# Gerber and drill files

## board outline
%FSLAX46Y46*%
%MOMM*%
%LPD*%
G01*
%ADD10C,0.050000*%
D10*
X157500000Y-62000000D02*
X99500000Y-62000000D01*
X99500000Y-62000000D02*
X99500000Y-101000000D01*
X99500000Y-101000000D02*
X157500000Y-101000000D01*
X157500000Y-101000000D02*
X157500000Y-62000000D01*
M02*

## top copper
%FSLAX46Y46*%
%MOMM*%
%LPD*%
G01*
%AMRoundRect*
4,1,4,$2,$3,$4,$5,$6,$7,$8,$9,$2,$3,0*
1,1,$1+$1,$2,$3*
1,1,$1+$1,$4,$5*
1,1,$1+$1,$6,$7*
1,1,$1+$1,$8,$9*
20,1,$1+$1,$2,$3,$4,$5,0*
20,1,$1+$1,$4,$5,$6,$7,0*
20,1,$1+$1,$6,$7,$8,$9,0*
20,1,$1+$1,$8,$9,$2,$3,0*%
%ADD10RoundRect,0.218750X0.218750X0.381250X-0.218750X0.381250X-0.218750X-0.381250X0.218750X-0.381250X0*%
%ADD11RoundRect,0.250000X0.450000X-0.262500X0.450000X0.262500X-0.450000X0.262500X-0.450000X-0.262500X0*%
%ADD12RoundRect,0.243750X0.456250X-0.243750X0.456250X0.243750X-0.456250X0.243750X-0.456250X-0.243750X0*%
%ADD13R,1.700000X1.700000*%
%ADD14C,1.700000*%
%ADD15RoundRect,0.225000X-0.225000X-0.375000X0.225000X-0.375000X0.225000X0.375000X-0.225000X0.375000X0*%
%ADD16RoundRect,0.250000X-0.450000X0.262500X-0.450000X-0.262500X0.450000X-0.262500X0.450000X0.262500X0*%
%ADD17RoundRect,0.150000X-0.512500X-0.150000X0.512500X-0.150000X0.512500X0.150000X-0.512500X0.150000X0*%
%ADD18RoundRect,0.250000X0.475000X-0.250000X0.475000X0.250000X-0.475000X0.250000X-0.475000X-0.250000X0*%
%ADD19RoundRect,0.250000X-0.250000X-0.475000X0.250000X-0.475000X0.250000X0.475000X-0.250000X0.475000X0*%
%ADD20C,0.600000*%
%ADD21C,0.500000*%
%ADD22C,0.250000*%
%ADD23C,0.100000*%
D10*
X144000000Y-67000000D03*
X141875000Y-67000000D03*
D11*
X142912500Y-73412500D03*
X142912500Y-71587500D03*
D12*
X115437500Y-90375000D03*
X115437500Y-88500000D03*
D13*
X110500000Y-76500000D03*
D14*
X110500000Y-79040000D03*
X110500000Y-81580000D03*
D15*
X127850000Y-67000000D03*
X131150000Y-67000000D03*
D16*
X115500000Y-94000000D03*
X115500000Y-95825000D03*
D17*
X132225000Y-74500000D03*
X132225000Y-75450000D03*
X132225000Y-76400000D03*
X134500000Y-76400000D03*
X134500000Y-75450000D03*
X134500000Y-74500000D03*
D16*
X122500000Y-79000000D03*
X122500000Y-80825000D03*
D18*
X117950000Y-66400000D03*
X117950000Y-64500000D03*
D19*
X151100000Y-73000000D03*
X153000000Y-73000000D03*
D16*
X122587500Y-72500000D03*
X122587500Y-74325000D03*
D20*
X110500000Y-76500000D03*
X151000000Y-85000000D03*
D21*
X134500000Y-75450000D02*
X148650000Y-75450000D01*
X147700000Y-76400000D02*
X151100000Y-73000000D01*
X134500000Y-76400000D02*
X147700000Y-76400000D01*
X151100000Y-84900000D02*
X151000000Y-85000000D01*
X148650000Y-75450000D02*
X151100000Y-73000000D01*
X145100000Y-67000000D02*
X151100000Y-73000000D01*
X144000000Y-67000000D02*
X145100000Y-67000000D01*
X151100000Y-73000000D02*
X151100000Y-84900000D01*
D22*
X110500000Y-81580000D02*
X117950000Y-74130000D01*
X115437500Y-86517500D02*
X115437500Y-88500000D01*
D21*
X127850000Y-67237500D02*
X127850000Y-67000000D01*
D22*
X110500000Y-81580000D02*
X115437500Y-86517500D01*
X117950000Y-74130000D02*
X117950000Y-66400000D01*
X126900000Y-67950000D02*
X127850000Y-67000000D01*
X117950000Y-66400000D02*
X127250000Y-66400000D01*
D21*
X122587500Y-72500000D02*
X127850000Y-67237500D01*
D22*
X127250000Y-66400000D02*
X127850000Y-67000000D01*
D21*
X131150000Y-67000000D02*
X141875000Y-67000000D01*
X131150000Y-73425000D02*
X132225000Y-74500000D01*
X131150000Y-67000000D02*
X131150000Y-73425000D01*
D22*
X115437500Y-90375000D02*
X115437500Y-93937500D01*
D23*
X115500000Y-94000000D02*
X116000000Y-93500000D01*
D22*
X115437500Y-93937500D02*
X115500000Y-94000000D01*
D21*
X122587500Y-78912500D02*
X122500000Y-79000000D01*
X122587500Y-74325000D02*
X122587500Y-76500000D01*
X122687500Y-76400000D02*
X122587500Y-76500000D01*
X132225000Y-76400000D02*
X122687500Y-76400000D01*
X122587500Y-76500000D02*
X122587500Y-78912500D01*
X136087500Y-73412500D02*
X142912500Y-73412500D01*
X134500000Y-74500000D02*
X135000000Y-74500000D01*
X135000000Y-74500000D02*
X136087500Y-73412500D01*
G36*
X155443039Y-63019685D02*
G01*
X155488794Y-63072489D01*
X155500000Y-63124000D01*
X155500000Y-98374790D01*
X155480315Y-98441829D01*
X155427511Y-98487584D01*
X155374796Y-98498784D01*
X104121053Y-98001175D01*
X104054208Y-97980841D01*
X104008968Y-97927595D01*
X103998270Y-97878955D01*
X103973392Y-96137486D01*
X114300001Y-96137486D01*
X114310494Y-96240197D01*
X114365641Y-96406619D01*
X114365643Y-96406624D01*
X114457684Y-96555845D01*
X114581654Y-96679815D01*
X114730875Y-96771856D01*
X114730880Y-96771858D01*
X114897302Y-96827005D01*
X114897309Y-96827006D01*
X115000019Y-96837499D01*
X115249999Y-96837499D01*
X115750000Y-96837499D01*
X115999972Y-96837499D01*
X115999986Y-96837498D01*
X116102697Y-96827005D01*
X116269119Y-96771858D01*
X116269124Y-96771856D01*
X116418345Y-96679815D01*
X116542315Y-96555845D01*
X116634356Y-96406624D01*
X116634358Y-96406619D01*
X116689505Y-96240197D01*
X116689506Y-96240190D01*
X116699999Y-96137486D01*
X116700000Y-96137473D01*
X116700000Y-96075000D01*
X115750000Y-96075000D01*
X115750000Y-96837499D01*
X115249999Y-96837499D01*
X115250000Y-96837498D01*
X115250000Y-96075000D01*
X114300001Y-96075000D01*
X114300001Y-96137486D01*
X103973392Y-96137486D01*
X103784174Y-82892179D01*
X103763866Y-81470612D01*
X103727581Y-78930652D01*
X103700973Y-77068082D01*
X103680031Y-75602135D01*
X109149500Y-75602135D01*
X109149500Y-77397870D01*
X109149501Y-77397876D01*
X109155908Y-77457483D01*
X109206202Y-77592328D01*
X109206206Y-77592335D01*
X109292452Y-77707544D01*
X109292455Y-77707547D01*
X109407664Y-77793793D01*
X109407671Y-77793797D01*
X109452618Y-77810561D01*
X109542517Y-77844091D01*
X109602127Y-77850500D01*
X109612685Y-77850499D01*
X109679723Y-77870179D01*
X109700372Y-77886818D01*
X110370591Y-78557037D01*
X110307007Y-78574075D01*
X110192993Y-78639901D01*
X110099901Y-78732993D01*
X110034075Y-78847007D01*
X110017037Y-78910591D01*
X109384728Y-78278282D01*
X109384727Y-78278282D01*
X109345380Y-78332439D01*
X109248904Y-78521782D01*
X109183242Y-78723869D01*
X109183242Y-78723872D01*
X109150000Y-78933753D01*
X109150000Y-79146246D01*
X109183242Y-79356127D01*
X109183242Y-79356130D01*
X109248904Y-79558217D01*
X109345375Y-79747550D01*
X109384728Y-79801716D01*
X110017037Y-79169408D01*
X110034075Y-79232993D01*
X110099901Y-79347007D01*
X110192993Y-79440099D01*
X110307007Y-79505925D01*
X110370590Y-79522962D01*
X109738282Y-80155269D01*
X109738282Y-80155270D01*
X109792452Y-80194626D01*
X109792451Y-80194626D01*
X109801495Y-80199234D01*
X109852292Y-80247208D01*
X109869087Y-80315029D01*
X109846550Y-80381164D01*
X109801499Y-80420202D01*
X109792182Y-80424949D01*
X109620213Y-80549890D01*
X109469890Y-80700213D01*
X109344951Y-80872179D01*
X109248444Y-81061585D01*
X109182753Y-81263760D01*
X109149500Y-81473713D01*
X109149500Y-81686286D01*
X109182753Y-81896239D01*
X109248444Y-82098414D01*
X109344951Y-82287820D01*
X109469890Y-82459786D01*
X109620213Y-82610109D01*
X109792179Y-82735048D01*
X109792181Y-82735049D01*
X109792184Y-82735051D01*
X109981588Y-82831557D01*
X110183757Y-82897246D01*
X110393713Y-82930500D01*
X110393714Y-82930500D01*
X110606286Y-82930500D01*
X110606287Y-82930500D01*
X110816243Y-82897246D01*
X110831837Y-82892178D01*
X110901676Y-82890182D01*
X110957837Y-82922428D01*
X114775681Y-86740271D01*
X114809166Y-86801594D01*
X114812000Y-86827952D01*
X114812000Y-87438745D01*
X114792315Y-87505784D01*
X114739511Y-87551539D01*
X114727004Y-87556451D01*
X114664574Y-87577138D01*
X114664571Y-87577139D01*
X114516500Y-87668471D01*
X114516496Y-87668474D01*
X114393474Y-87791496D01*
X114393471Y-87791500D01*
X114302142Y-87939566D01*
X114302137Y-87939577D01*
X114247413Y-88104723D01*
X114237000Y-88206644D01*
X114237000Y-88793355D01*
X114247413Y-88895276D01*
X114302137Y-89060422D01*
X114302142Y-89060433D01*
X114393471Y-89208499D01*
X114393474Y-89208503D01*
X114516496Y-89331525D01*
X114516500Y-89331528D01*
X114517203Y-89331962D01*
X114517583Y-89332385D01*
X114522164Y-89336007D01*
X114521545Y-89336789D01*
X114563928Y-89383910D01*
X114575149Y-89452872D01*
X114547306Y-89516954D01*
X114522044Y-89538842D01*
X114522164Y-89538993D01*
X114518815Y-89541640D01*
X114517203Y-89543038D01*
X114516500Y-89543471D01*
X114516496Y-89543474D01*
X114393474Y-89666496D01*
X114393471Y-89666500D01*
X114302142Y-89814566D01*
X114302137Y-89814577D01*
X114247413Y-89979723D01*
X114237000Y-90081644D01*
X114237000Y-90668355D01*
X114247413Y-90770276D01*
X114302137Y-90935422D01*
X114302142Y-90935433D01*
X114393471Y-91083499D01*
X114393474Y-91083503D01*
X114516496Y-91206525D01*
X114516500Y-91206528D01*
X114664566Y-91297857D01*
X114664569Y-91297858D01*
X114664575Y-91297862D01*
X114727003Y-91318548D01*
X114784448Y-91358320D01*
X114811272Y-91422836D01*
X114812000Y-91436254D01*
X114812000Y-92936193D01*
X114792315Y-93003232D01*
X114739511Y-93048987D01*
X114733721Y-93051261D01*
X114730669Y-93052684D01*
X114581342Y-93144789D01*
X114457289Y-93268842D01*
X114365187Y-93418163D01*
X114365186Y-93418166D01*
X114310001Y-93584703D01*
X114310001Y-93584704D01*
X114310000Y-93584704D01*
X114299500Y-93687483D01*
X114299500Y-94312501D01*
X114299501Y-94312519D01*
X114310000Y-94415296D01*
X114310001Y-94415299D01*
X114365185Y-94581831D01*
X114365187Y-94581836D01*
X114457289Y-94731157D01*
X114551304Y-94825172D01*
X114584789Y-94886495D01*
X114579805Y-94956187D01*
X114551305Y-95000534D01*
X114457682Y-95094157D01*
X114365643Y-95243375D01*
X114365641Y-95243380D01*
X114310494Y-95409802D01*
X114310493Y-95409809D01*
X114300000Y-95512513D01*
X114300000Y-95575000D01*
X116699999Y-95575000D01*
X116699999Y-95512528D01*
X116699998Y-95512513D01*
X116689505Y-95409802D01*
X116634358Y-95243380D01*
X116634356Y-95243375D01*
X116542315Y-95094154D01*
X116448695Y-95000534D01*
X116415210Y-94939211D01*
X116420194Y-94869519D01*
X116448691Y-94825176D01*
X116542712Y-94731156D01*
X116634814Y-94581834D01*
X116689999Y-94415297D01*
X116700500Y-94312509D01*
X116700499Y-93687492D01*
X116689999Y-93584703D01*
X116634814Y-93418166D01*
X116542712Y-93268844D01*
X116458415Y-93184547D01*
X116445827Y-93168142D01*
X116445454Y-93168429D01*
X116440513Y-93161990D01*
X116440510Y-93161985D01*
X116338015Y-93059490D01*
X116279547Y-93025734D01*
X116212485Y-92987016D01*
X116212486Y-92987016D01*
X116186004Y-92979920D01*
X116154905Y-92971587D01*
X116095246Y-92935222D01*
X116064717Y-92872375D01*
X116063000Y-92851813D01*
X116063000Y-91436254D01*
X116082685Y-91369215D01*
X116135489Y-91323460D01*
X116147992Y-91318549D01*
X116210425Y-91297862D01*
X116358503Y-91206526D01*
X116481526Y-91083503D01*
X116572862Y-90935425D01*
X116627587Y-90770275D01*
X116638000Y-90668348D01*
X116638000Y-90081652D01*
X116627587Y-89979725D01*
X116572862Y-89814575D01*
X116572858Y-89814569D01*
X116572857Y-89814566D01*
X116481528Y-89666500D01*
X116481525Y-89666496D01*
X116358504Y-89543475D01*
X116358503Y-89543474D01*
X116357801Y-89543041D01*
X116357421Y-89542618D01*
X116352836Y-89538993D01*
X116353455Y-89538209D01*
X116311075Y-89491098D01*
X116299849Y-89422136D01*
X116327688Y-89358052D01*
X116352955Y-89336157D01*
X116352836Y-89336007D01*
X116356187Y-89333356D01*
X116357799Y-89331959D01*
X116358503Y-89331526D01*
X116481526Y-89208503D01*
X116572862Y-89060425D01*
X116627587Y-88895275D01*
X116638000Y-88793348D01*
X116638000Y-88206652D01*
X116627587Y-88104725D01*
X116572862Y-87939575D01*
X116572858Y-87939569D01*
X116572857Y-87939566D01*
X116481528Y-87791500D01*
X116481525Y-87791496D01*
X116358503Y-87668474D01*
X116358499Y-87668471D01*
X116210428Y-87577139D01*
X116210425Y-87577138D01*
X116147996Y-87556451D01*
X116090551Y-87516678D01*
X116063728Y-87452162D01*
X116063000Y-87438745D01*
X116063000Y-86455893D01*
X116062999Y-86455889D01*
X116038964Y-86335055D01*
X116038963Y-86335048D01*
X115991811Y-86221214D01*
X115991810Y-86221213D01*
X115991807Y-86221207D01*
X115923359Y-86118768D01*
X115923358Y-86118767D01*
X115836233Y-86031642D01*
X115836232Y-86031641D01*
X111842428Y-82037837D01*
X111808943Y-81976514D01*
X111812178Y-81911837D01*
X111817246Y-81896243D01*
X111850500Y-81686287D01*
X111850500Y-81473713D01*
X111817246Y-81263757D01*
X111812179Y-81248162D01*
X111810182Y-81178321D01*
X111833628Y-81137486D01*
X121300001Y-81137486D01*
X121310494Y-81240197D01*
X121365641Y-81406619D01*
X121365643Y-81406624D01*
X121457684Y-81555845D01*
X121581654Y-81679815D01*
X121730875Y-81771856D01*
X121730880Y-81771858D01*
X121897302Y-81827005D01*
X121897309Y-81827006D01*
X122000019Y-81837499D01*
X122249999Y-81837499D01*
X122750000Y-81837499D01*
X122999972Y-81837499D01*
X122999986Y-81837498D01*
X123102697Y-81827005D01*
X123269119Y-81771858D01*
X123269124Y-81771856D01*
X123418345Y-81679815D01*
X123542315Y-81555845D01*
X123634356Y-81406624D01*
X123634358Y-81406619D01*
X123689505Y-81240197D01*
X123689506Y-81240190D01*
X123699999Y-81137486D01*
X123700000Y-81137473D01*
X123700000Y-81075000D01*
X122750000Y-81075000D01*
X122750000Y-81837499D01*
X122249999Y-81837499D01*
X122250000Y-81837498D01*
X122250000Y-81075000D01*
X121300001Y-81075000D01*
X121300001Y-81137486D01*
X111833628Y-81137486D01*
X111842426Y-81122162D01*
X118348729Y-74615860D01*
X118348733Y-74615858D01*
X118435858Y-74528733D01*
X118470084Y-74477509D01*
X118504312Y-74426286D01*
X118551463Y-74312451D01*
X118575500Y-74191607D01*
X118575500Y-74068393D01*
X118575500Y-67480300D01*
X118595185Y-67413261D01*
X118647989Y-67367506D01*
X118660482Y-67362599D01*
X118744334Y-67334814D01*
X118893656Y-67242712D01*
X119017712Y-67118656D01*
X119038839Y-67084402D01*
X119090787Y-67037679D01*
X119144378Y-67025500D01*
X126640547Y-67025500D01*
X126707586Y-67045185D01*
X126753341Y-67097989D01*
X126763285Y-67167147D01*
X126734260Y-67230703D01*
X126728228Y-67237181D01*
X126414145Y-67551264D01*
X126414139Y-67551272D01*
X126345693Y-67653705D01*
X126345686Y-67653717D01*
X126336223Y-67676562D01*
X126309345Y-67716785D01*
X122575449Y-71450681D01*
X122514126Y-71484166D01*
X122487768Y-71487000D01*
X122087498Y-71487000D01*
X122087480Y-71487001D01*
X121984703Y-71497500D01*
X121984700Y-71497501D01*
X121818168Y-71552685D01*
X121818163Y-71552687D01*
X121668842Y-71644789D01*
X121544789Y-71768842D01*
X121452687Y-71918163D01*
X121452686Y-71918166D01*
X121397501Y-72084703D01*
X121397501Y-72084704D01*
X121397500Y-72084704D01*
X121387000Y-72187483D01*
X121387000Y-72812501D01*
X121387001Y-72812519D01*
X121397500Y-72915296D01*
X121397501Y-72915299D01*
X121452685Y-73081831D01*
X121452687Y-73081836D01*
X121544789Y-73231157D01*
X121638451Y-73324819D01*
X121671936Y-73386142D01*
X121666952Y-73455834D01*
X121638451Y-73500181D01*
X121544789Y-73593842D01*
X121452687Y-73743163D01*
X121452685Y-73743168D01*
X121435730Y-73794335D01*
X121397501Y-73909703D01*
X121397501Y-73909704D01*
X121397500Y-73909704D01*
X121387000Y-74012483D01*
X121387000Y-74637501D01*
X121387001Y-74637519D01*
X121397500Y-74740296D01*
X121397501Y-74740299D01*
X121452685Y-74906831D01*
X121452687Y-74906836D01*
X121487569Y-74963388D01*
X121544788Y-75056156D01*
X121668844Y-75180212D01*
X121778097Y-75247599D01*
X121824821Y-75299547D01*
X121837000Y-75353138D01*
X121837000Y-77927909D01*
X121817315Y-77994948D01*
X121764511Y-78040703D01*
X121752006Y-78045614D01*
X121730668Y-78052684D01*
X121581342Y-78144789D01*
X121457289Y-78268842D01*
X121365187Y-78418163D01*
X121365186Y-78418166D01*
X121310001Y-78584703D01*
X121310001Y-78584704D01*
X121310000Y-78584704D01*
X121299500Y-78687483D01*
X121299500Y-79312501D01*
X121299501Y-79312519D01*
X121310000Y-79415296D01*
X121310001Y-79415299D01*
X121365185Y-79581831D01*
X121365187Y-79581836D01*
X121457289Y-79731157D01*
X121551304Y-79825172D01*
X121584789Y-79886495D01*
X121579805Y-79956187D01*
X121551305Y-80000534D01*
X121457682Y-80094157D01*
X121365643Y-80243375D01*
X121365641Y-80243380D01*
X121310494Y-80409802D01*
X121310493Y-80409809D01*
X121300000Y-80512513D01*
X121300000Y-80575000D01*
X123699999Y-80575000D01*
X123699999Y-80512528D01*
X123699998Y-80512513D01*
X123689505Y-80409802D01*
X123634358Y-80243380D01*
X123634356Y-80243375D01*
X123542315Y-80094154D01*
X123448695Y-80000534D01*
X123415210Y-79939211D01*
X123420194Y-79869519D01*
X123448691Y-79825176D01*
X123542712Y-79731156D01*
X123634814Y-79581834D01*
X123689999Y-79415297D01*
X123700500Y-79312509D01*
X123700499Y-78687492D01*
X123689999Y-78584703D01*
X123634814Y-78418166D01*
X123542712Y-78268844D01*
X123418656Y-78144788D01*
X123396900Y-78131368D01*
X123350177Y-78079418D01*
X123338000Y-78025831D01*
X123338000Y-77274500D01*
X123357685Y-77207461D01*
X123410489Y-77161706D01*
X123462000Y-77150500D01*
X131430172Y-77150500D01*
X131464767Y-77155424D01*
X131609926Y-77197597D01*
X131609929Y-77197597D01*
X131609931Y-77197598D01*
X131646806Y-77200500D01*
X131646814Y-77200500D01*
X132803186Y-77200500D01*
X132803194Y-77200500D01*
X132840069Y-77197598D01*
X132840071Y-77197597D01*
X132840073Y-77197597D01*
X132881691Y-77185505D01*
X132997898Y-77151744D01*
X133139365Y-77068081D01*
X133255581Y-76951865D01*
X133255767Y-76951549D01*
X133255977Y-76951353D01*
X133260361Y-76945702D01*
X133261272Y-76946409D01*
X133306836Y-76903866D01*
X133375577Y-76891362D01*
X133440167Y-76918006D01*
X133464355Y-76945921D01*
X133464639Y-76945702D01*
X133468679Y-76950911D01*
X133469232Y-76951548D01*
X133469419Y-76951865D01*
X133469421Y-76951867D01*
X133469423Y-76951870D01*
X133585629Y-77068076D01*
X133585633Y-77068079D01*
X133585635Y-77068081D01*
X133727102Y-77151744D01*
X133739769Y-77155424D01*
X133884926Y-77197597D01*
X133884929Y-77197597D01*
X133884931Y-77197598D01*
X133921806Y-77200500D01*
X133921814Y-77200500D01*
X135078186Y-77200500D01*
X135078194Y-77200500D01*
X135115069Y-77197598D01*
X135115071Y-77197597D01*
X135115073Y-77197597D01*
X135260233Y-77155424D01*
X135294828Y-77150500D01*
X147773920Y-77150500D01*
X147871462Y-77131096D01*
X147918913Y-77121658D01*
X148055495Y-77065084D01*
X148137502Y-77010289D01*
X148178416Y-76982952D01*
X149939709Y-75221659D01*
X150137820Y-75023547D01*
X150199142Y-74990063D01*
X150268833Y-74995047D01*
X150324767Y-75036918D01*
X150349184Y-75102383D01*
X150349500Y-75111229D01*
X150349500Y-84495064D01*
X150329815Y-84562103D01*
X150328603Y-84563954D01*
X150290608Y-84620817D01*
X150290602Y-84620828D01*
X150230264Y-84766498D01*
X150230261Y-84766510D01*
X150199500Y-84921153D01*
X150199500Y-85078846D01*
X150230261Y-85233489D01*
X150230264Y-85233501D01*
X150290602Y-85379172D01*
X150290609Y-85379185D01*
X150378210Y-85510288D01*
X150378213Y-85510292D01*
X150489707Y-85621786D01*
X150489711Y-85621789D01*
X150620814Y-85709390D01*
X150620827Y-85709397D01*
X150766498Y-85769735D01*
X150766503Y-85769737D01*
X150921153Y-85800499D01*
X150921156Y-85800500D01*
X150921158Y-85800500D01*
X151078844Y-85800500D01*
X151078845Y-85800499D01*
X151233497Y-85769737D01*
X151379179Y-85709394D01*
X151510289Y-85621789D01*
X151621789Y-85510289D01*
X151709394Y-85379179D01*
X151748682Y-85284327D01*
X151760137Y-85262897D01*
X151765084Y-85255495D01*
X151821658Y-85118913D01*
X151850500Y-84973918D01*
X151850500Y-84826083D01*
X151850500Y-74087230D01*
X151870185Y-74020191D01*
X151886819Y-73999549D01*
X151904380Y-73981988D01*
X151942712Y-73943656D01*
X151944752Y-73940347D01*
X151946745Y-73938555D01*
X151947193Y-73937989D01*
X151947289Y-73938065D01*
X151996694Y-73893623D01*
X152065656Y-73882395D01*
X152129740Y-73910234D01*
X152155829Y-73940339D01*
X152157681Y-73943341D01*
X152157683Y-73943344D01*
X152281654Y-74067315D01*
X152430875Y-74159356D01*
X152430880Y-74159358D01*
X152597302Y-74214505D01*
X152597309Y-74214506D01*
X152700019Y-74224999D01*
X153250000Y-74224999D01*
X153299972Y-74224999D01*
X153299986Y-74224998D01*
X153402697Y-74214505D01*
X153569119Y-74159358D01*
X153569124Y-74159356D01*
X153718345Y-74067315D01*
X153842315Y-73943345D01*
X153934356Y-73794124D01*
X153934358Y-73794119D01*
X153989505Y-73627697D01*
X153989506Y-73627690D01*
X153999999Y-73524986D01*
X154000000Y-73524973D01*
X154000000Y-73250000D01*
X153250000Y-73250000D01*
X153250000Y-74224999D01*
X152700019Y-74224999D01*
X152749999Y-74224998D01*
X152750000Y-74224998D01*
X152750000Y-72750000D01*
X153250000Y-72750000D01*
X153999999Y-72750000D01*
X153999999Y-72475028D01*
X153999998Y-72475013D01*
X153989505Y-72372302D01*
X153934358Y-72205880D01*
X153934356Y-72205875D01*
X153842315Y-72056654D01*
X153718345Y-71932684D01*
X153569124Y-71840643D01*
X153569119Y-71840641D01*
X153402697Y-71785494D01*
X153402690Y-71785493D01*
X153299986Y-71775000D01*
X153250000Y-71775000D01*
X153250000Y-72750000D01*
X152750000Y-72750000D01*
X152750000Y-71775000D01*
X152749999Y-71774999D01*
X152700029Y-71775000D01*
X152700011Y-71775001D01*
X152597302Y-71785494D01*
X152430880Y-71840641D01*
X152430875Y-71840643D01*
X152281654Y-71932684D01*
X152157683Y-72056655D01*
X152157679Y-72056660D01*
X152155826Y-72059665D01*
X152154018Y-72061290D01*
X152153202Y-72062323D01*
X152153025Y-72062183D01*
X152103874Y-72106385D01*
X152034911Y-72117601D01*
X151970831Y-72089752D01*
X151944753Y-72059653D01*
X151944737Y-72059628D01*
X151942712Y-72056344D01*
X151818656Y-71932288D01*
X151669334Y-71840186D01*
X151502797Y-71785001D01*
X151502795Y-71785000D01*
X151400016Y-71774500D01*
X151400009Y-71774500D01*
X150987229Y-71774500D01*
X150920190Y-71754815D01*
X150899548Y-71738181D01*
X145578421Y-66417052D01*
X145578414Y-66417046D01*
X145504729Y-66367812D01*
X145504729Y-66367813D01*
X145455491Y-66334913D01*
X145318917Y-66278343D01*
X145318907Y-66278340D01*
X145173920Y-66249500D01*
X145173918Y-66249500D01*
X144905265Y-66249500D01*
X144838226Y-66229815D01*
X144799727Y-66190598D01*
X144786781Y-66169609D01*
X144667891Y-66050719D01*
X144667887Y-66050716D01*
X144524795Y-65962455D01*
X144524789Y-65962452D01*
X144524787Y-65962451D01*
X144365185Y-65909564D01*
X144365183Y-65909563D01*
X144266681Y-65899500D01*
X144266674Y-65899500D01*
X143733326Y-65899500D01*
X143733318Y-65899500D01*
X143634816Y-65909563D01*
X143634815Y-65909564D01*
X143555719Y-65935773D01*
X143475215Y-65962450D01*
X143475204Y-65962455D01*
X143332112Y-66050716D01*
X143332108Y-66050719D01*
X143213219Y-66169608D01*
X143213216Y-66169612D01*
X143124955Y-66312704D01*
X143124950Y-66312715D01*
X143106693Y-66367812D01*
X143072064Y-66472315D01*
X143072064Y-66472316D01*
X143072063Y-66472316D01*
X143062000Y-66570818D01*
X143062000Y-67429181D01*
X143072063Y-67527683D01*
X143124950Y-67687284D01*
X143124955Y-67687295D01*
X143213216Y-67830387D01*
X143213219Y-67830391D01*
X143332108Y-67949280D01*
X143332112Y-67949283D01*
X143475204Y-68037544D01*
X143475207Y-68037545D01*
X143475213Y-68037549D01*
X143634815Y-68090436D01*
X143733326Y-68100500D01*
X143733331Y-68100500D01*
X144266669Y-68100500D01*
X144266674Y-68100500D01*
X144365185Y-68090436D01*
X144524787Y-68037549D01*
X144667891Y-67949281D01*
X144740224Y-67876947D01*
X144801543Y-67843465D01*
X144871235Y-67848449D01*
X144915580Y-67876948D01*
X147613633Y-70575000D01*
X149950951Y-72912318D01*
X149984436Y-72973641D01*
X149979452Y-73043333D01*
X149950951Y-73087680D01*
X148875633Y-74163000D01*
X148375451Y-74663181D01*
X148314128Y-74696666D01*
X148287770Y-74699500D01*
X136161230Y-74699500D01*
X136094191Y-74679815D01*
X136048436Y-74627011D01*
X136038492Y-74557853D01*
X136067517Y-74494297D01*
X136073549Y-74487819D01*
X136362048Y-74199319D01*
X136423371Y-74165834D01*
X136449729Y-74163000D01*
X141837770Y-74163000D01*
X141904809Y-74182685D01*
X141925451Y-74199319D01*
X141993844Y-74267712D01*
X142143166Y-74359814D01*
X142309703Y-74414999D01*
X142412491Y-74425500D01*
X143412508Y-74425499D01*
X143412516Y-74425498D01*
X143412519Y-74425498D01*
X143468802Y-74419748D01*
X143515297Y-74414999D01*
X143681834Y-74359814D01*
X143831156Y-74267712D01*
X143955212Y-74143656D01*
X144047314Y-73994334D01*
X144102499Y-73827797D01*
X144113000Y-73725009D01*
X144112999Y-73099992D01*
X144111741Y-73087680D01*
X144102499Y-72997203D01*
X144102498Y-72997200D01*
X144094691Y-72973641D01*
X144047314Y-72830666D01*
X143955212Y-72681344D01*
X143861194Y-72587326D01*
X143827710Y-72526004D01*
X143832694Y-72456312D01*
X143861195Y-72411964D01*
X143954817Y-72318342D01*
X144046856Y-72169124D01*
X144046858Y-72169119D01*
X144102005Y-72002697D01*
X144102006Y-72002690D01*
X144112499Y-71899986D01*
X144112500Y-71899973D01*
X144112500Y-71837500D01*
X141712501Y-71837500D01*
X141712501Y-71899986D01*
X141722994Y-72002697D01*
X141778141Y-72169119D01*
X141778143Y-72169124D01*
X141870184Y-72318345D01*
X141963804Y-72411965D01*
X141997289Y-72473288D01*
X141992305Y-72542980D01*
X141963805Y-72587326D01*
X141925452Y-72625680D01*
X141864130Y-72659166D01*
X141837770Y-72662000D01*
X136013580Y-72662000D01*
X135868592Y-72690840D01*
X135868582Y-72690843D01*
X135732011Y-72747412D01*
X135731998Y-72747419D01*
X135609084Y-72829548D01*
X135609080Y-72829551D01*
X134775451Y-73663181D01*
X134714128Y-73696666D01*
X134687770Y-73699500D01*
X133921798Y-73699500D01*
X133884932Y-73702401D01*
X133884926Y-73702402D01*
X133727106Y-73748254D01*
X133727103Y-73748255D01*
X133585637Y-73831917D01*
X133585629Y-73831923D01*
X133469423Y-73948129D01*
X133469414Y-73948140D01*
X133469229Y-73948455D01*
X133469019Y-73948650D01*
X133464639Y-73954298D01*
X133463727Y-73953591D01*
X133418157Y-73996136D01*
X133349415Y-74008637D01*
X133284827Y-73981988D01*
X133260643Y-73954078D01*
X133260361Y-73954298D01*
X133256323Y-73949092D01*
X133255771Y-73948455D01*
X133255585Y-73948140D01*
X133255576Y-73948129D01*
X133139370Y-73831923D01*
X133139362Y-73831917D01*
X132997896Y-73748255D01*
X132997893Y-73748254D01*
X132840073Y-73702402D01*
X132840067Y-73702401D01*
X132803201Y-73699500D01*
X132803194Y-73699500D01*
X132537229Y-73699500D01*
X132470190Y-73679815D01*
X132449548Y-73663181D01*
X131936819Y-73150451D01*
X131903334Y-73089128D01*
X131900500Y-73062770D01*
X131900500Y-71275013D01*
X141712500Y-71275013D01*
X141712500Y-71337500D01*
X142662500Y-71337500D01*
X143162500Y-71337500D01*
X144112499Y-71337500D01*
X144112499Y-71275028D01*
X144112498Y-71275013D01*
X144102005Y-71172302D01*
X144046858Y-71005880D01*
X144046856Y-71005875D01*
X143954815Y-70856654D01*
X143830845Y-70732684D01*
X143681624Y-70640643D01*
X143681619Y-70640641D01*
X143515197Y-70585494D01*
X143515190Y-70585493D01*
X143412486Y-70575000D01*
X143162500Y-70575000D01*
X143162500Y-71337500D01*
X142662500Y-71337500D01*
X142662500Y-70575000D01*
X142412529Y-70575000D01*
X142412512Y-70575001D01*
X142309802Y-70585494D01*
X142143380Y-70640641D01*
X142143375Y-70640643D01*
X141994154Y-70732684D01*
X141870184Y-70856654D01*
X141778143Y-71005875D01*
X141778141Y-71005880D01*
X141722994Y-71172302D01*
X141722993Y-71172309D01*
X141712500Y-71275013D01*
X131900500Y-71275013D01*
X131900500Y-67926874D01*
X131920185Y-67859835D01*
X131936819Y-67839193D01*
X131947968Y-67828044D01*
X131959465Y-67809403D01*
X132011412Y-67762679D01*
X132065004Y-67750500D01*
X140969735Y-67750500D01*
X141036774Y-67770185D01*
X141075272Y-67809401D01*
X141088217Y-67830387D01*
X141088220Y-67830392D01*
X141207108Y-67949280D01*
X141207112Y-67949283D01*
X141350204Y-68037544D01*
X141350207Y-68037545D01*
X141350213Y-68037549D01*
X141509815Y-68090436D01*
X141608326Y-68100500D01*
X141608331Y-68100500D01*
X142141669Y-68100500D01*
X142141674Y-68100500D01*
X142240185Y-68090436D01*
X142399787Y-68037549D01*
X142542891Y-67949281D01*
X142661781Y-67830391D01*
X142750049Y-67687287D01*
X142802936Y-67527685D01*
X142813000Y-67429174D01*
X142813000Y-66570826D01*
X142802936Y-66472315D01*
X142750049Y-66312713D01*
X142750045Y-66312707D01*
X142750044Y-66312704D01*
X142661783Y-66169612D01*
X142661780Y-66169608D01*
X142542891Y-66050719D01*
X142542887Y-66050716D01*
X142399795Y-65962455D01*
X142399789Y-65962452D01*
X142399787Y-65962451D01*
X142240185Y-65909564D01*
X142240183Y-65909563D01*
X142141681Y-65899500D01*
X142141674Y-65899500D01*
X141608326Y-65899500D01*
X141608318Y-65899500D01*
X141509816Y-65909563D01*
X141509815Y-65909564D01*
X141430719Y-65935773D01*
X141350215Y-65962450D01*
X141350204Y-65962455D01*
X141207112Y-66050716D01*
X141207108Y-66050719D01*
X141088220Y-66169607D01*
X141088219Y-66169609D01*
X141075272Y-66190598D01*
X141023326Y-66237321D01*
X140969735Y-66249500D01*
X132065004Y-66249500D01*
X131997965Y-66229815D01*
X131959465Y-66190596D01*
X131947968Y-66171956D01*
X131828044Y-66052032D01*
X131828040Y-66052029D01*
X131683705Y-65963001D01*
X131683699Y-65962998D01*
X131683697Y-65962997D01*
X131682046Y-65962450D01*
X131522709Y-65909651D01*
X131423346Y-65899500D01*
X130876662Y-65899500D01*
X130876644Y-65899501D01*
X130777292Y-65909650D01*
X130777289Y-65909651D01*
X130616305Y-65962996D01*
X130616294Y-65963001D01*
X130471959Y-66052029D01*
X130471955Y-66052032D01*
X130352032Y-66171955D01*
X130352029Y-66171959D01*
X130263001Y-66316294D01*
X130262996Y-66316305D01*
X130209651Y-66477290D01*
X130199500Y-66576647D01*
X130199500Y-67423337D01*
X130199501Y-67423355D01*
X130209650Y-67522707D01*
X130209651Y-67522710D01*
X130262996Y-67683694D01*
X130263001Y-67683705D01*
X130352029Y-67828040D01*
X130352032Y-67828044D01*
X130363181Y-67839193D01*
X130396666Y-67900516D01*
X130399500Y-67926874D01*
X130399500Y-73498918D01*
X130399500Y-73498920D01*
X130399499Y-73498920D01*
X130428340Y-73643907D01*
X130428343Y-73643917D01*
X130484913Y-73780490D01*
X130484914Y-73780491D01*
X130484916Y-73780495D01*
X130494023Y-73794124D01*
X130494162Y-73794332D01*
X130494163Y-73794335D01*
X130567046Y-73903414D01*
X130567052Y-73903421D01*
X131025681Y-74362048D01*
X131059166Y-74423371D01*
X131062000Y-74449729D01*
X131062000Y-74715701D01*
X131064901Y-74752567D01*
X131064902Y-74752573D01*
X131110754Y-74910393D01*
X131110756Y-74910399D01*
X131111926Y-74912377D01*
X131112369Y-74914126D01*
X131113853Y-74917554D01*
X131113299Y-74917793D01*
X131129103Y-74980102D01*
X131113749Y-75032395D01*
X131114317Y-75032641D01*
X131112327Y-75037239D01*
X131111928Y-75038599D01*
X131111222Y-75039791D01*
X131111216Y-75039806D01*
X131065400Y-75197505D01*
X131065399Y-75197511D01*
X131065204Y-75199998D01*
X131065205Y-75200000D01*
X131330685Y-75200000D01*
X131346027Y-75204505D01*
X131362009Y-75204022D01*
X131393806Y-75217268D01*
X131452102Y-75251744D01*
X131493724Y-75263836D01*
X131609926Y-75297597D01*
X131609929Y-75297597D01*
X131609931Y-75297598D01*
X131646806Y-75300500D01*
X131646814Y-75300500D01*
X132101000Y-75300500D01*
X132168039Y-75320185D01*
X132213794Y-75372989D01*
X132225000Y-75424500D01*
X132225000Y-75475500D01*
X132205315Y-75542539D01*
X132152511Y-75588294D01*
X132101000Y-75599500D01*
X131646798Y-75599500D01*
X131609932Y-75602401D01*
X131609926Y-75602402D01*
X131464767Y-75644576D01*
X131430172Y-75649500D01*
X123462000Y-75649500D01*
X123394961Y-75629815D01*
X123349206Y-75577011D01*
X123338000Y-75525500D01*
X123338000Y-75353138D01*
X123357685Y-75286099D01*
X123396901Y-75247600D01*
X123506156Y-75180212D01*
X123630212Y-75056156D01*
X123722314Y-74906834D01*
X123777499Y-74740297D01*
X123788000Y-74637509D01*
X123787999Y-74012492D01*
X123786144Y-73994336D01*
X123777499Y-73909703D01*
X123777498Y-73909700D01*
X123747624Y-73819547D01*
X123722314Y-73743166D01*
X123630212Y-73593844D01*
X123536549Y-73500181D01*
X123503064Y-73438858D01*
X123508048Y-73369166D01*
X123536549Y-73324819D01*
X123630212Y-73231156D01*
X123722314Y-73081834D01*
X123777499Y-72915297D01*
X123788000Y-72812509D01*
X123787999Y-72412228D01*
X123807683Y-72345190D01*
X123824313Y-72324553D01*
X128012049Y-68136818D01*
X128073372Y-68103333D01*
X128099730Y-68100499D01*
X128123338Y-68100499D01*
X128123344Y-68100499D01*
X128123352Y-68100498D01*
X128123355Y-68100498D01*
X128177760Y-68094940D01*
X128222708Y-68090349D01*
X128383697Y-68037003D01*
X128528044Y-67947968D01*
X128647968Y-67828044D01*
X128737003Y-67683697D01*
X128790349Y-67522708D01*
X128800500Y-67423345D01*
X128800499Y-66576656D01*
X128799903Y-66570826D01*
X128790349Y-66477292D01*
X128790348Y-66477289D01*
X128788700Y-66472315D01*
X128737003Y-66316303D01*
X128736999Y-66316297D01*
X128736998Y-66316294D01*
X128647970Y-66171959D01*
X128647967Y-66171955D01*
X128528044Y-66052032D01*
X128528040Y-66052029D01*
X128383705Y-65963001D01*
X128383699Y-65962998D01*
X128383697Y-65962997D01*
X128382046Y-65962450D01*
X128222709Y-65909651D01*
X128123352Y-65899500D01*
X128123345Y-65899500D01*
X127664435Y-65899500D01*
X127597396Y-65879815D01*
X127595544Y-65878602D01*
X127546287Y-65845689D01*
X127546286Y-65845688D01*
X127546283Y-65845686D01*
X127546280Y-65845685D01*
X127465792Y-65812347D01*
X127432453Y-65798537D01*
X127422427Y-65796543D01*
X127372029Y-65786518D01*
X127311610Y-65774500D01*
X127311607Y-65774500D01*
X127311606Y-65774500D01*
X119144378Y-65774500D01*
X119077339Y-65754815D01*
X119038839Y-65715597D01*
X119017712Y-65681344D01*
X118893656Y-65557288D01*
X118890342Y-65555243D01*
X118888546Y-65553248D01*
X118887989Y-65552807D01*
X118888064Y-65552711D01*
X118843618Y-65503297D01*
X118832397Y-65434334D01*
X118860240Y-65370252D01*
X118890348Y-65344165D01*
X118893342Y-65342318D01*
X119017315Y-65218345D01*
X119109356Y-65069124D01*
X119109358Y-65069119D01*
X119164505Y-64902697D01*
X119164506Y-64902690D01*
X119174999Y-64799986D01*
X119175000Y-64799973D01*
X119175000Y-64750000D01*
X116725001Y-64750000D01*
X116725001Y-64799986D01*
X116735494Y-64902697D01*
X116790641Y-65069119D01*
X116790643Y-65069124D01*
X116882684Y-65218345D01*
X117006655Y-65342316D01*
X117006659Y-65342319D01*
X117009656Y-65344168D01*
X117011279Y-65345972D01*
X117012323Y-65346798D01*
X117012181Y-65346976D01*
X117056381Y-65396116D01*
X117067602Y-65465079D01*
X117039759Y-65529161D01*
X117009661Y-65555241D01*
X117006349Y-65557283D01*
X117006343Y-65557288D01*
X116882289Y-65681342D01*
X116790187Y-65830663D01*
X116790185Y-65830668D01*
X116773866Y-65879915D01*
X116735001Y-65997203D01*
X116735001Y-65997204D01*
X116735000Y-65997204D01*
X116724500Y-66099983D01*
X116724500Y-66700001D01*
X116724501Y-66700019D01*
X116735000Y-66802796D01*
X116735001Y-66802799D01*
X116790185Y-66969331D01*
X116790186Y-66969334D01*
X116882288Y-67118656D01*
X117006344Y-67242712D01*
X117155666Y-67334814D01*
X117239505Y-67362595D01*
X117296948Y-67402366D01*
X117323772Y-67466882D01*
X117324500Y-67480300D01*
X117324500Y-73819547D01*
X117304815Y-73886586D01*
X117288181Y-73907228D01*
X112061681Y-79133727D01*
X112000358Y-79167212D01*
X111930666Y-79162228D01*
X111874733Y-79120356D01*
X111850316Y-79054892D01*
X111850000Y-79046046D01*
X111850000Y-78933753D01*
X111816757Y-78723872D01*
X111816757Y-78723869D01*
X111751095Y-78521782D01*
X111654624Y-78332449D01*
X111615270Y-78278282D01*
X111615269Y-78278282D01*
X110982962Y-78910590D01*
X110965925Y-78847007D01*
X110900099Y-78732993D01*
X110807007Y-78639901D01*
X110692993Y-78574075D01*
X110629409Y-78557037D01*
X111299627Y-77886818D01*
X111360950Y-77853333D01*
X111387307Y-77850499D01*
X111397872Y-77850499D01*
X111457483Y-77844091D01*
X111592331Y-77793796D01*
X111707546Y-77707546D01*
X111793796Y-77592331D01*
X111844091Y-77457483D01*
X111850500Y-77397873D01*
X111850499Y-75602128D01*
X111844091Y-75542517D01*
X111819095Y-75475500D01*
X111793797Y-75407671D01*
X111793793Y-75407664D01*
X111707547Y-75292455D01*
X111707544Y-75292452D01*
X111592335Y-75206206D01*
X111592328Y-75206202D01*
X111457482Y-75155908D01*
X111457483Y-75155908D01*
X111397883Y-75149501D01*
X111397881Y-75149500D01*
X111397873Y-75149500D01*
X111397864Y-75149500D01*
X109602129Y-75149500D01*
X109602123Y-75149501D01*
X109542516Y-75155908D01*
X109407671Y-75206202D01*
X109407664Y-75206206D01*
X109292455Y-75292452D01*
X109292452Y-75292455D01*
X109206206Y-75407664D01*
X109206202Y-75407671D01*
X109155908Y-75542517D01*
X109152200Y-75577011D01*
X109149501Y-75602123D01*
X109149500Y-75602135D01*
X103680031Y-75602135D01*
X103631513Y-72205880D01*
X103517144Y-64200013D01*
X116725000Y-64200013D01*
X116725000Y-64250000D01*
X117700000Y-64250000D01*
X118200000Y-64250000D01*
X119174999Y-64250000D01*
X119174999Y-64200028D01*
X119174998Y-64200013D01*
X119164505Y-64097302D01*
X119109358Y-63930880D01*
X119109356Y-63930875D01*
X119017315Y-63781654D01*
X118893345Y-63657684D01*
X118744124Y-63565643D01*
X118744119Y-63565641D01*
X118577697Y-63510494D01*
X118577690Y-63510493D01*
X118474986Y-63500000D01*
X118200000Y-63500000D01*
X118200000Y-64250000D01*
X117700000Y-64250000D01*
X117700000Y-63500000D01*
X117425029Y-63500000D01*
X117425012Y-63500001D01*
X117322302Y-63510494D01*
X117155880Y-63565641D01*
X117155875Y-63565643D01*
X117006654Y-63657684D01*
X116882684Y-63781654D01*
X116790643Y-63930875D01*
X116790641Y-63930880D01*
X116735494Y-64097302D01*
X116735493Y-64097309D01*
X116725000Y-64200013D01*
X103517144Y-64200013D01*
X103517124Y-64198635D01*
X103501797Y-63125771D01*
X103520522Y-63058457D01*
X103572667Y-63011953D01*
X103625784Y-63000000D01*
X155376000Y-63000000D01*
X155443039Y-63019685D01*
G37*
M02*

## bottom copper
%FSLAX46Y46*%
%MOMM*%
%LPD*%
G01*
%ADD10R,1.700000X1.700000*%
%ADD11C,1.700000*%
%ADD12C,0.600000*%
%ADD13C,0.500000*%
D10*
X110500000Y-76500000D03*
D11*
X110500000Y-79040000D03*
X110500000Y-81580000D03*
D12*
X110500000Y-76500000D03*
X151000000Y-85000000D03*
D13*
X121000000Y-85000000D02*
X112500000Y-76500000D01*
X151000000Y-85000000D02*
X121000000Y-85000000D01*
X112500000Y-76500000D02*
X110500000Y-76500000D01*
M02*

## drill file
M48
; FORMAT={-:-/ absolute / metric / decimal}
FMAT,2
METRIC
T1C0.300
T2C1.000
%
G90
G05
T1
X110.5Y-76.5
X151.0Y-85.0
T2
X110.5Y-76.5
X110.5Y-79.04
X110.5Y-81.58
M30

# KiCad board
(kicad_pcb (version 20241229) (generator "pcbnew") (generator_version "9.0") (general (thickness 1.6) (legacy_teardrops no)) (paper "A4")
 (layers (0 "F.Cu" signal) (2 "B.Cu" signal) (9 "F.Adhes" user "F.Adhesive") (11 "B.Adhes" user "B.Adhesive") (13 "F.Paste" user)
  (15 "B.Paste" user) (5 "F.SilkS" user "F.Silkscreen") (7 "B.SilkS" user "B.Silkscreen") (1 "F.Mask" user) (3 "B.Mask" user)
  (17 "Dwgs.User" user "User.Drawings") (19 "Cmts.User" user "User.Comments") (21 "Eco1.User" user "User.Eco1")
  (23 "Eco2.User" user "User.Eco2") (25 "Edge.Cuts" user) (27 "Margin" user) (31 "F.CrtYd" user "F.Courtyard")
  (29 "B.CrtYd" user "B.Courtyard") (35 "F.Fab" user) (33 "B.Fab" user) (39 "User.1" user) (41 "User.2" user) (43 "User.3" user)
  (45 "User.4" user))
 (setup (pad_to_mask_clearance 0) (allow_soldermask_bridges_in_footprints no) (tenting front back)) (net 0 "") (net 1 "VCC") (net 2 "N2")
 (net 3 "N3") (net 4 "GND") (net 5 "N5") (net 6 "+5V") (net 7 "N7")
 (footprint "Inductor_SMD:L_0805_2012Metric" (layer "F.Cu") (at 142.9375 67 180)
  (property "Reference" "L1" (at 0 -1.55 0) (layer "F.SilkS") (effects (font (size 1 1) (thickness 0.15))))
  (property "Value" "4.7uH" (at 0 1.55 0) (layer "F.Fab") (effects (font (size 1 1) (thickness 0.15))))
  (pad "1" smd roundrect (at -1.0625 0 180) (size 0.875 1.2) (layers "F.Cu" "F.Mask" "F.Paste") (roundrect_rratio 0.25) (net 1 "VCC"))
  (pad "2" smd roundrect (at 1.0625 0 180) (size 0.875 1.2) (layers "F.Cu" "F.Mask" "F.Paste") (roundrect_rratio 0.25) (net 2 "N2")))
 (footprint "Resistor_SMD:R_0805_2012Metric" (layer "F.Cu") (at 142.9125 72.5 90)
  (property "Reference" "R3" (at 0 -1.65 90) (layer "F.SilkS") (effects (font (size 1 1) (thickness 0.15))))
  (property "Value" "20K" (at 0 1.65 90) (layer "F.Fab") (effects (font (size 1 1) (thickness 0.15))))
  (pad "1" smd roundrect (at -0.9125 0 90) (size 1.025 1.4) (layers "F.Cu" "F.Mask" "F.Paste") (roundrect_rratio 0.243902) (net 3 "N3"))
  (pad "2" smd roundrect (at 0.9125 0 90) (size 1.025 1.4) (layers "F.Cu" "F.Mask" "F.Paste") (roundrect_rratio 0.243902) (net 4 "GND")))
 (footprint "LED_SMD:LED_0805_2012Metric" (layer "F.Cu") (at 115.4375 89.4375 90)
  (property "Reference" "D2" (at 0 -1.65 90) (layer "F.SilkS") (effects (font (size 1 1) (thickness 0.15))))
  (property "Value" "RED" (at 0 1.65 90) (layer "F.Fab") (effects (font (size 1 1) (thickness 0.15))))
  (pad "1" smd roundrect (at -0.9375 0 90) (size 0.975 1.4) (layers "F.Cu" "F.Mask" "F.Paste") (roundrect_rratio 0.25) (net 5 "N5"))
  (pad "2" smd roundrect (at 0.9375 0 90) (size 0.975 1.4) (layers "F.Cu" "F.Mask" "F.Paste") (roundrect_rratio 0.25) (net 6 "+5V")))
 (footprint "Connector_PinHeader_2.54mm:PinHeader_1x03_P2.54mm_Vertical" (layer "F.Cu") (at 110.5 76.5)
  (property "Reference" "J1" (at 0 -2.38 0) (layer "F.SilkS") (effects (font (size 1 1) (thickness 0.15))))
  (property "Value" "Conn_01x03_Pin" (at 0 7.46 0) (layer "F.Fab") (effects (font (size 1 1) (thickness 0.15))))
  (pad "1" thru_hole rect (at 0 0) (size 1.7 1.7) (drill 1) (layers "*.Cu" "*.Mask") (remove_unused_layers no) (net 1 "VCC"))
  (pad "2" thru_hole circle (at 0 2.54) (size 1.7 1.7) (drill 1) (layers "*.Cu" "*.Mask") (remove_unused_layers no) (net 4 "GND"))
  (pad "3" thru_hole circle (at 0 5.08) (size 1.7 1.7) (drill 1) (layers "*.Cu" "*.Mask") (remove_unused_layers no) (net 6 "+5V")))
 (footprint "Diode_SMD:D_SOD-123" (layer "F.Cu") (at 129.5 67)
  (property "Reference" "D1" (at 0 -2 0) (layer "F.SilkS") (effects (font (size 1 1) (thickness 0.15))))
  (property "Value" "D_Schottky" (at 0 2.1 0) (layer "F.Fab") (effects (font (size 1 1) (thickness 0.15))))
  (pad "1" smd roundrect (at -1.65 0) (size 0.9 1.2) (layers "F.Cu" "F.Mask" "F.Paste") (roundrect_rratio 0.25) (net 6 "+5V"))
  (pad "2" smd roundrect (at 1.65 0) (size 0.9 1.2) (layers "F.Cu" "F.Mask" "F.Paste") (roundrect_rratio 0.25) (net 2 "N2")))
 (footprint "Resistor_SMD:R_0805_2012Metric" (layer "F.Cu") (at 115.5 94.9125 -90)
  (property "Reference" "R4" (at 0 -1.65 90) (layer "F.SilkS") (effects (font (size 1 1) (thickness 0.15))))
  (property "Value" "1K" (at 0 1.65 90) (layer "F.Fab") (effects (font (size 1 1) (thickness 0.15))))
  (pad "1" smd roundrect (at -0.9125 0 270) (size 1.025 1.4) (layers "F.Cu" "F.Mask" "F.Paste") (roundrect_rratio 0.243902) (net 5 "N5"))
  (pad "2" smd roundrect (at 0.9125 0 270) (size 1.025 1.4) (layers "F.Cu" "F.Mask" "F.Paste") (roundrect_rratio 0.243902) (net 4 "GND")))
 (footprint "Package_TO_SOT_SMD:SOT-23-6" (layer "F.Cu") (at 133.3625 75.45)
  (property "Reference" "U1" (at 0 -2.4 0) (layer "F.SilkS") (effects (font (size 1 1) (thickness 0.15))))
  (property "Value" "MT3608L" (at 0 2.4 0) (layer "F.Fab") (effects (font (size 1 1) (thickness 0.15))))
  (pad "1" smd roundrect (at -1.1375 -0.95) (size 1.325 0.6) (layers "F.Cu" "F.Mask" "F.Paste") (roundrect_rratio 0.25) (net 2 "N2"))
  (pad "2" smd roundrect (at -1.1375 0) (size 1.325 0.6) (layers "F.Cu" "F.Mask" "F.Paste") (roundrect_rratio 0.25) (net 4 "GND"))
  (pad "3" smd roundrect (at -1.1375 0.95) (size 1.325 0.6) (layers "F.Cu" "F.Mask" "F.Paste") (roundrect_rratio 0.25) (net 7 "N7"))
  (pad "4" smd roundrect (at 1.1375 0.95) (size 1.325 0.6) (layers "F.Cu" "F.Mask" "F.Paste") (roundrect_rratio 0.25) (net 1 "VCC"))
  (pad "5" smd roundrect (at 1.1375 0) (size 1.325 0.6) (layers "F.Cu" "F.Mask" "F.Paste") (roundrect_rratio 0.25) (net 1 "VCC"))
  (pad "6" smd roundrect (at 1.1375 -0.95) (size 1.325 0.6) (layers "F.Cu" "F.Mask" "F.Paste") (roundrect_rratio 0.25) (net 3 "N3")))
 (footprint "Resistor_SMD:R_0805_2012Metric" (layer "F.Cu") (at 122.5 79.9125 -90)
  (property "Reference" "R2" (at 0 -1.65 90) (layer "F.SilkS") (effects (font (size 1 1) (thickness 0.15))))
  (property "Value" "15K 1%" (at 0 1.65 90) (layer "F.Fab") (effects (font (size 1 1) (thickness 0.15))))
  (pad "1" smd roundrect (at -0.9125 0 270) (size 1.025 1.4) (layers "F.Cu" "F.Mask" "F.Paste") (roundrect_rratio 0.243902) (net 7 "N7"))
  (pad "2" smd roundrect (at 0.9125 0 270) (size 1.025 1.4) (layers "F.Cu" "F.Mask" "F.Paste") (roundrect_rratio 0.243902) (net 4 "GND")))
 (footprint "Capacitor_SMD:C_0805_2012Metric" (layer "F.Cu") (at 117.95 65.45 90)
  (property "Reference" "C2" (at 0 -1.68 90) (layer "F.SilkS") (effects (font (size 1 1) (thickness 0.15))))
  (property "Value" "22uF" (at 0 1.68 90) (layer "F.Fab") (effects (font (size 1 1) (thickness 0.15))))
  (pad "1" smd roundrect (at -0.95 0 90) (size 1 1.45) (layers "F.Cu" "F.Mask" "F.Paste") (roundrect_rratio 0.25) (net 6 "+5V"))
  (pad "2" smd roundrect (at 0.95 0 90) (size 1 1.45) (layers "F.Cu" "F.Mask" "F.Paste") (roundrect_rratio 0.25) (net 4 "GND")))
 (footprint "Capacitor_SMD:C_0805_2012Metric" (layer "F.Cu") (at 152.05 73)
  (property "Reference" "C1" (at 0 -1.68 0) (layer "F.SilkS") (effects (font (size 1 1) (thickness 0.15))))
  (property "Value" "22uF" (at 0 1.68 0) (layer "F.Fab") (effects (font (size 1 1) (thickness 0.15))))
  (pad "1" smd roundrect (at -0.95 0) (size 1 1.45) (layers "F.Cu" "F.Mask" "F.Paste") (roundrect_rratio 0.25) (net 1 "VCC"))
  (pad "2" smd roundrect (at 0.95 0) (size 1 1.45) (layers "F.Cu" "F.Mask" "F.Paste") (roundrect_rratio 0.25) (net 4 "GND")))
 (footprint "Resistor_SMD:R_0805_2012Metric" (layer "F.Cu") (at 122.5875 73.4125 -90)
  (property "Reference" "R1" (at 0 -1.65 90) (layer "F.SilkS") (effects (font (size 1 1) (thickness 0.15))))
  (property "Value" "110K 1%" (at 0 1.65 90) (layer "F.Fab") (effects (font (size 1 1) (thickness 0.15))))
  (pad "1" smd roundrect (at -0.9125 0 270) (size 1.025 1.4) (layers "F.Cu" "F.Mask" "F.Paste") (roundrect_rratio 0.243902) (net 6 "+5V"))
  (pad "2" smd roundrect (at 0.9125 0 270) (size 1.025 1.4) (layers "F.Cu" "F.Mask" "F.Paste") (roundrect_rratio 0.243902) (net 7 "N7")))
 (gr_line (start 157.5 62) (end 99.5 62) (stroke (width 0.05) (type default)) (layer "Edge.Cuts"))
 (gr_line (start 99.5 62) (end 99.5 101) (stroke (width 0.05) (type default)) (layer "Edge.Cuts"))
 (gr_line (start 99.5 101) (end 157.5 101) (stroke (width 0.05) (type default)) (layer "Edge.Cuts"))
 (gr_line (start 157.5 101) (end 157.5 62) (stroke (width 0.05) (type default)) (layer "Edge.Cuts"))
 (segment (start 134.5 75.45) (end 148.65 75.45) (width 0.5) (layer "F.Cu") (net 1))
 (segment (start 147.7 76.4) (end 151.1 73) (width 0.5) (layer "F.Cu") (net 1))
 (segment (start 134.5 76.4) (end 147.7 76.4) (width 0.5) (layer "F.Cu") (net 1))
 (segment (start 151.1 84.9) (end 151 85) (width 0.5) (layer "F.Cu") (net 1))
 (segment (start 148.65 75.45) (end 151.1 73) (width 0.5) (layer "F.Cu") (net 1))
 (segment (start 145.1 67) (end 151.1 73) (width 0.5) (layer "F.Cu") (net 1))
 (segment (start 144 67) (end 145.1 67) (width 0.5) (layer "F.Cu") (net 1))
 (segment (start 151.1 73) (end 151.1 84.9) (width 0.5) (layer "F.Cu") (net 1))
 (via (at 110.5 76.5) (size 0.6) (drill 0.3) (layers "F.Cu" "B.Cu") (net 1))
 (via (at 151 85) (size 0.6) (drill 0.3) (layers "F.Cu" "B.Cu") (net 1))
 (segment (start 121 85) (end 112.5 76.5) (width 0.5) (layer "B.Cu") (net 1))
 (segment (start 151 85) (end 121 85) (width 0.5) (layer "B.Cu") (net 1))
 (segment (start 112.5 76.5) (end 110.5 76.5) (width 0.5) (layer "B.Cu") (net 1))
 (segment (start 110.5 81.58) (end 117.95 74.13) (width 0.25) (layer "F.Cu") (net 6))
 (segment (start 115.4375 86.5175) (end 115.4375 88.5) (width 0.25) (layer "F.Cu") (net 6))
 (segment (start 127.85 67.2375) (end 127.85 67) (width 0.5) (layer "F.Cu") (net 6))
 (segment (start 110.5 81.58) (end 115.4375 86.5175) (width 0.25) (layer "F.Cu") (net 6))
 (segment (start 117.95 74.13) (end 117.95 66.4) (width 0.25) (layer "F.Cu") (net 6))
 (segment (start 126.9 67.95) (end 127.85 67) (width 0.25) (layer "F.Cu") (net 6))
 (segment (start 117.95 66.4) (end 127.25 66.4) (width 0.25) (layer "F.Cu") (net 6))
 (segment (start 122.5875 72.5) (end 127.85 67.2375) (width 0.5) (layer "F.Cu") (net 6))
 (segment (start 127.25 66.4) (end 127.85 67) (width 0.25) (layer "F.Cu") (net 6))
 (segment (start 131.15 67) (end 141.875 67) (width 0.5) (layer "F.Cu") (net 2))
 (segment (start 131.15 73.425) (end 132.225 74.5) (width 0.5) (layer "F.Cu") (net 2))
 (segment (start 131.15 67) (end 131.15 73.425) (width 0.5) (layer "F.Cu") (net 2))
 (segment (start 115.4375 90.375) (end 115.4375 93.9375) (width 0.25) (layer "F.Cu") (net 5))
 (segment (start 115.5 94) (end 116 93.5) (width 0.1) (layer "F.Cu") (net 5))
 (segment (start 115.4375 93.9375) (end 115.5 94) (width 0.25) (layer "F.Cu") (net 5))
 (segment (start 122.5875 78.9125) (end 122.5 79) (width 0.5) (layer "F.Cu") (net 7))
 (segment (start 122.5875 74.325) (end 122.5875 76.5) (width 0.5) (layer "F.Cu") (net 7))
 (segment (start 122.6875 76.4) (end 122.5875 76.5) (width 0.5) (layer "F.Cu") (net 7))
 (segment (start 132.225 76.4) (end 122.6875 76.4) (width 0.5) (layer "F.Cu") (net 7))
 (segment (start 122.5875 76.5) (end 122.5875 78.9125) (width 0.5) (layer "F.Cu") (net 7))
 (segment (start 136.0875 73.4125) (end 142.9125 73.4125) (width 0.5) (layer "F.Cu") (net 3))
 (segment (start 134.5 74.5) (end 135 74.5) (width 0.5) (layer "F.Cu") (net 3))
 (segment (start 135 74.5) (end 136.0875 73.4125) (width 0.5) (layer "F.Cu") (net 3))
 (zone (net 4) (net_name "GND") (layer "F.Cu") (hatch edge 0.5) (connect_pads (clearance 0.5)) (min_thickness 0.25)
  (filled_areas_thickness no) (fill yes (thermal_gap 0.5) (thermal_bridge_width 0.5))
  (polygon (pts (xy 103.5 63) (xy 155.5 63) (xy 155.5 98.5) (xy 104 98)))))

